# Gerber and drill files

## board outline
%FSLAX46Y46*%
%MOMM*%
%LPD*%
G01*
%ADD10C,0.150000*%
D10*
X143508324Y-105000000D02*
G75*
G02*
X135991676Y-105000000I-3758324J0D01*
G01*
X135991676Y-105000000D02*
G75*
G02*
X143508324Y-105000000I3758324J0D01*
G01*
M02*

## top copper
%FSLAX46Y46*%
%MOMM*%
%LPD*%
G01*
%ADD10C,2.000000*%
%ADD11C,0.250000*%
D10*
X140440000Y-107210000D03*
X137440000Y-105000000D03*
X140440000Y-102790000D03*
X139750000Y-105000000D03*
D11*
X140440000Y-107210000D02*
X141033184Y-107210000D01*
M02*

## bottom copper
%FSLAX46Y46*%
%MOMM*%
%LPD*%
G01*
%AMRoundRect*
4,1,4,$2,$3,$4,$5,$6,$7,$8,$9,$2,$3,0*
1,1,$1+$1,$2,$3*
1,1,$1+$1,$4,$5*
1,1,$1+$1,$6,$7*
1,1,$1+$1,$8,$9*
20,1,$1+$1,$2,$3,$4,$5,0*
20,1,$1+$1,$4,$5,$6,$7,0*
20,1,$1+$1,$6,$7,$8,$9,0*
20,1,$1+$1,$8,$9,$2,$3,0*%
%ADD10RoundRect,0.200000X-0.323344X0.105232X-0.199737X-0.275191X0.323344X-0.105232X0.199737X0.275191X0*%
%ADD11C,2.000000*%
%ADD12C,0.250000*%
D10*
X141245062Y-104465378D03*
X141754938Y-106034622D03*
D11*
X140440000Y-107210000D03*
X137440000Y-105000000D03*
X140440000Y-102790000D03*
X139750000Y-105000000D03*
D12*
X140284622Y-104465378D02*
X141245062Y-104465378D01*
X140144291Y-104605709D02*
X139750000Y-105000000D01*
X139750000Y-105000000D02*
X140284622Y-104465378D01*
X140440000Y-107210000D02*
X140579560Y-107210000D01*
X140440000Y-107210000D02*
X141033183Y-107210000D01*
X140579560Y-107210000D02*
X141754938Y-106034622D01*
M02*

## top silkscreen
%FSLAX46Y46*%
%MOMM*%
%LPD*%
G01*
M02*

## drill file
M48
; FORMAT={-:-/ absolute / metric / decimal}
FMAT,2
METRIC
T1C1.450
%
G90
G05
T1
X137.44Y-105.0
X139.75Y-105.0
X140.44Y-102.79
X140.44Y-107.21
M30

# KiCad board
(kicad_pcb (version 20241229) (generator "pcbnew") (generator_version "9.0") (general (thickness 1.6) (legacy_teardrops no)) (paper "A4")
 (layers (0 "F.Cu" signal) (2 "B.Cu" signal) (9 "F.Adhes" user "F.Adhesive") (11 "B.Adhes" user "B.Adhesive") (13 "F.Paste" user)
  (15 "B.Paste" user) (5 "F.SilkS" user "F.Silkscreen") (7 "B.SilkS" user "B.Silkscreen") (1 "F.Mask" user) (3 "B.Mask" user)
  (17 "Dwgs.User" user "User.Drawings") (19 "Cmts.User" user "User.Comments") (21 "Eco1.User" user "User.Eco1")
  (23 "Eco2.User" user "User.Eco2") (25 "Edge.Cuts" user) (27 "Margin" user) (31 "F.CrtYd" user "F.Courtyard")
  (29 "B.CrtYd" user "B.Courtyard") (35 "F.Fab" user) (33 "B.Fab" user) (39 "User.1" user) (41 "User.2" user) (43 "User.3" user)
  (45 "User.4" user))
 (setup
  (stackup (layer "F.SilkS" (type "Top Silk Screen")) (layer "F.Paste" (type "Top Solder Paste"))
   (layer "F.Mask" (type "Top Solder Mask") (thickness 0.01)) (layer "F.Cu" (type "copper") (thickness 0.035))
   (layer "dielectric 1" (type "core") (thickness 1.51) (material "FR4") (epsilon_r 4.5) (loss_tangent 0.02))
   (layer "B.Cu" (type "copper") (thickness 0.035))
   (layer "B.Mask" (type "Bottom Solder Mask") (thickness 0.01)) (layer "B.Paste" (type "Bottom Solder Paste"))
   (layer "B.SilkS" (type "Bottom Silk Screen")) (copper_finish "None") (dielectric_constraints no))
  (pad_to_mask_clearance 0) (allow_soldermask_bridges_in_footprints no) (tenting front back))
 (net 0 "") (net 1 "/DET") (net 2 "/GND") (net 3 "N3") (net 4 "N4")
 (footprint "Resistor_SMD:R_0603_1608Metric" (layer "B.Cu") (at 141.5 105.25 -72)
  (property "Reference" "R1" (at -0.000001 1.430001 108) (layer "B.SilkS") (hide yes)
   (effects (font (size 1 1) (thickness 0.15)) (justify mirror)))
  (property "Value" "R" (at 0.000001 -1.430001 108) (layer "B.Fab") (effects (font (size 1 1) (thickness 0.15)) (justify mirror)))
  (pad "1" smd roundrect (at -0.825 -0.000001 288) (size 0.8 0.95) (layers "B.Cu" "B.Mask" "B.Paste") (roundrect_rratio 0.25) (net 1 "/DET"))
  (pad "2" smd roundrect (at 0.825 0.000001 288) (size 0.8 0.95) (layers "B.Cu" "B.Mask" "B.Paste") (roundrect_rratio 0.25) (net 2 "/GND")))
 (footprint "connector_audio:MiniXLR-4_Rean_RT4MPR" (layer "B.Cu") (at 139.75 105 90)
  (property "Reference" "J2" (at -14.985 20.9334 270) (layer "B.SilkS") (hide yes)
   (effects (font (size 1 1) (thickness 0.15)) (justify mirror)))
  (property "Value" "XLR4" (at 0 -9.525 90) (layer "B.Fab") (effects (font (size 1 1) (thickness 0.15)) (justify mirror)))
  (pad "1" thru_hole circle (at -2.21 0.69 270) (size 2 2) (drill 1.45) (layers "*.Cu" "*.Mask") (remove_unused_layers no) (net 2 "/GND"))
  (pad "2" thru_hole circle (at 0 -2.31 270) (size 2 2) (drill 1.45) (layers "*.Cu" "*.Mask") (remove_unused_layers no) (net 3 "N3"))
  (pad "3" thru_hole circle (at 2.21 0.69 270) (size 2 2) (drill 1.45) (layers "*.Cu" "*.Mask") (remove_unused_layers no) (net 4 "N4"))
  (pad "4" thru_hole circle (at 0 0 270) (size 2 2) (drill 1.45) (layers "*.Cu" "*.Mask") (remove_unused_layers no) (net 1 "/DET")))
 (gr_circle (center 139.75 105) (end 143.5 105.25) (stroke (width 0.15) (type default)) (fill no) (layer "Edge.Cuts"))
 (segment (start 140.284622 104.465378) (end 141.245062 104.465378) (width 0.25) (layer "B.Cu") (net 1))
 (segment (start 140.144291 104.605709) (end 139.75 105) (width 0.25) (layer "B.Cu") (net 1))
 (segment (start 139.75 105) (end 140.284622 104.465378) (width 0.25) (layer "B.Cu") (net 1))
 (segment (start 140.44 107.21) (end 141.033184 107.21) (width 0.25) (layer "F.Cu") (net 2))
 (segment (start 140.44 107.21) (end 140.57956 107.21) (width 0.25) (layer "B.Cu") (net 2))
 (segment (start 140.44 107.21) (end 141.033183 107.21) (width 0.25) (layer "B.Cu") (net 2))
 (segment (start 140.57956 107.21) (end 141.754938 106.034622) (width 0.25) (layer "B.Cu") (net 2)))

